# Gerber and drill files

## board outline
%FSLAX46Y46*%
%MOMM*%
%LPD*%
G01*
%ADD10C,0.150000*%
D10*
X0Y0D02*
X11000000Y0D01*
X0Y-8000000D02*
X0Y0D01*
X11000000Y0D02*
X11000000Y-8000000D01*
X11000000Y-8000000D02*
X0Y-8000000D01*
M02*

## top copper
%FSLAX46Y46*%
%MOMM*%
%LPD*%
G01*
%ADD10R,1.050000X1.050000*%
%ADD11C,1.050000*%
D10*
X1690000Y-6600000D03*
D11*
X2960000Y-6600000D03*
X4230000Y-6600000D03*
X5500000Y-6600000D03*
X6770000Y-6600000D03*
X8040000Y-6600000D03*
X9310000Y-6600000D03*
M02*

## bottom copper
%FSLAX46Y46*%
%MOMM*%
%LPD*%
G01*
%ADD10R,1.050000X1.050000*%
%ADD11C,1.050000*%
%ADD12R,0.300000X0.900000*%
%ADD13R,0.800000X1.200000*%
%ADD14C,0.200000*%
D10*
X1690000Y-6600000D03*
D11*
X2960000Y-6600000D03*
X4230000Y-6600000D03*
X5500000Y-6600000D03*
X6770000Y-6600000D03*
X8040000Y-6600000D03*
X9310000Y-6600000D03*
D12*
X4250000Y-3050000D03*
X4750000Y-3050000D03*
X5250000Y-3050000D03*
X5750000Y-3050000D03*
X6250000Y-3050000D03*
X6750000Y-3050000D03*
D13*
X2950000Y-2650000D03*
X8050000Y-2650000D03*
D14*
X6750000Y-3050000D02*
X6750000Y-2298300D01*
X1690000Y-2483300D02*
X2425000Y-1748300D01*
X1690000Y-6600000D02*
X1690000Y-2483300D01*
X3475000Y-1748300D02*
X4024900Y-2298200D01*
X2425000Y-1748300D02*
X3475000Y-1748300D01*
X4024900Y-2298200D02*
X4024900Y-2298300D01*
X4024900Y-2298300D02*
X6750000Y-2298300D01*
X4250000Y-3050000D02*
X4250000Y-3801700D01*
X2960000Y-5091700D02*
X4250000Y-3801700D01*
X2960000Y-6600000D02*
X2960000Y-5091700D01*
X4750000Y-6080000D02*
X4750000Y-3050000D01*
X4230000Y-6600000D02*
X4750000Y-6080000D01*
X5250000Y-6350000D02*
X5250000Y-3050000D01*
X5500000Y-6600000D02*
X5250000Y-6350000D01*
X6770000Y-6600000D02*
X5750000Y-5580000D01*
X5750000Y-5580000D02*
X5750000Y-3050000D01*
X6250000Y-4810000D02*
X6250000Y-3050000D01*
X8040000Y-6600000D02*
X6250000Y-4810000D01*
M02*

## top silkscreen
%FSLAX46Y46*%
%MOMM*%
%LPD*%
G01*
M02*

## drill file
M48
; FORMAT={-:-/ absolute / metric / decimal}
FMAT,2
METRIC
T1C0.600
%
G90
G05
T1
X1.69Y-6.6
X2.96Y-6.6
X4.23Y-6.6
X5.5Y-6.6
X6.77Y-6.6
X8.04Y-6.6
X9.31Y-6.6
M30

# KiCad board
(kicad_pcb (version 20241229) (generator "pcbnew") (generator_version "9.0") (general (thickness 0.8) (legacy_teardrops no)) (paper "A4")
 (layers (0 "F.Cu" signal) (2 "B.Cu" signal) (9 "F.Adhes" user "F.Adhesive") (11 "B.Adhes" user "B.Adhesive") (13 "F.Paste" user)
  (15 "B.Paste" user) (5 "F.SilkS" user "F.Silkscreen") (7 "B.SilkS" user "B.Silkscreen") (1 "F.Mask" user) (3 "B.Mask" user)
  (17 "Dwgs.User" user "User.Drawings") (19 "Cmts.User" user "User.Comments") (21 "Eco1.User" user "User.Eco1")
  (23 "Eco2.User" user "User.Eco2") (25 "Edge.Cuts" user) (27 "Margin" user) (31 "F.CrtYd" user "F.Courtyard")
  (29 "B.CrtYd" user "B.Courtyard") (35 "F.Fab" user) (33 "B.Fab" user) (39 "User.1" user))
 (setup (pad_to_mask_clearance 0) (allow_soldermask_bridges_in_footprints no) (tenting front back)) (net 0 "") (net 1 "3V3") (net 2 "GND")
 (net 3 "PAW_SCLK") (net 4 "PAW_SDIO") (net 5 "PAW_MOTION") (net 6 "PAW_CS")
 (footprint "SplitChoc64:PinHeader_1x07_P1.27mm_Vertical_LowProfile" (layer "F.Cu") (at 0 0)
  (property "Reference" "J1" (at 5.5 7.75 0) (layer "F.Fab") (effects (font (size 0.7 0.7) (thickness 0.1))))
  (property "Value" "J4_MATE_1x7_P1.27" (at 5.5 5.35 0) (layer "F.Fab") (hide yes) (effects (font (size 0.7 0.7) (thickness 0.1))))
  (pad "1" thru_hole rect (at 1.69 6.6) (size 1.05 1.05) (drill 0.6) (layers "*.Cu" "*.Mask") (remove_unused_layers no) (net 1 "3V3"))
  (pad "2" thru_hole circle (at 2.96 6.6) (size 1.05 1.05) (drill 0.6) (layers "*.Cu" "*.Mask") (remove_unused_layers no) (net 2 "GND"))
  (pad "3" thru_hole circle (at 4.23 6.6) (size 1.05 1.05) (drill 0.6) (layers "*.Cu" "*.Mask") (remove_unused_layers no) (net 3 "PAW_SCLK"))
  (pad "4" thru_hole circle (at 5.5 6.6) (size 1.05 1.05) (drill 0.6) (layers "*.Cu" "*.Mask") (remove_unused_layers no) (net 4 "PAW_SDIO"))
  (pad "5" thru_hole circle (at 6.77 6.6) (size 1.05 1.05) (drill 0.6) (layers "*.Cu" "*.Mask") (remove_unused_layers no)
   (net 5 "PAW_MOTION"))
  (pad "6" thru_hole circle (at 8.04 6.6) (size 1.05 1.05) (drill 0.6) (layers "*.Cu" "*.Mask") (remove_unused_layers no) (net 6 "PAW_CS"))
  (pad "7" thru_hole circle (at 9.31 6.6) (size 1.05 1.05) (drill 0.6) (layers "*.Cu" "*.Mask") (remove_unused_layers no)))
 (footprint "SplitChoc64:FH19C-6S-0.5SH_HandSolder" (layer "B.Cu") (at 0 0)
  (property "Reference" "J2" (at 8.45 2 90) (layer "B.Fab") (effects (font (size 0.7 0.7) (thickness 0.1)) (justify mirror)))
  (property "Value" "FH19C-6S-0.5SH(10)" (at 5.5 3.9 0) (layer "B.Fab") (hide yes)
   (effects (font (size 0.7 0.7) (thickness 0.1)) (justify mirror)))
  (pad "1" smd rect (at 4.25 3.05) (size 0.3 0.9) (layers "B.Cu" "B.Mask" "B.Paste") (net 2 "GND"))
  (pad "2" smd rect (at 4.75 3.05) (size 0.3 0.9) (layers "B.Cu" "B.Mask" "B.Paste") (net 3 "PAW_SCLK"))
  (pad "3" smd rect (at 5.25 3.05) (size 0.3 0.9) (layers "B.Cu" "B.Mask" "B.Paste") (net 4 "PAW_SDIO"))
  (pad "4" smd rect (at 5.75 3.05) (size 0.3 0.9) (layers "B.Cu" "B.Mask" "B.Paste") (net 5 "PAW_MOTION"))
  (pad "5" smd rect (at 6.25 3.05) (size 0.3 0.9) (layers "B.Cu" "B.Mask" "B.Paste") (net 6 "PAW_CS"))
  (pad "6" smd rect (at 6.75 3.05) (size 0.3 0.9) (layers "B.Cu" "B.Mask" "B.Paste") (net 1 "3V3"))
  (pad "MP" smd rect (at 2.95 2.65) (size 0.8 1.2) (layers "B.Cu" "B.Mask" "B.Paste"))
  (pad "MP" smd rect (at 8.05 2.65) (size 0.8 1.2) (layers "B.Cu" "B.Mask" "B.Paste")))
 (gr_line (start 0 0) (end 11 0) (stroke (width 0.15) (type default)) (layer "Edge.Cuts"))
 (gr_line (start 0 8) (end 0 0) (stroke (width 0.15) (type default)) (layer "Edge.Cuts"))
 (gr_line (start 11 0) (end 11 8) (stroke (width 0.15) (type default)) (layer "Edge.Cuts"))
 (gr_line (start 11 8) (end 0 8) (stroke (width 0.15) (type default)) (layer "Edge.Cuts"))
 (segment (start 6.75 3.05) (end 6.75 2.2983) (width 0.2) (layer "B.Cu") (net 1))
 (segment (start 1.69 2.4833) (end 2.425 1.7483) (width 0.2) (layer "B.Cu") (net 1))
 (segment (start 1.69 6.6) (end 1.69 2.4833) (width 0.2) (layer "B.Cu") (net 1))
 (segment (start 3.475 1.7483) (end 4.0249 2.2982) (width 0.2) (layer "B.Cu") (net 1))
 (segment (start 2.425 1.7483) (end 3.475 1.7483) (width 0.2) (layer "B.Cu") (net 1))
 (segment (start 4.0249 2.2982) (end 4.0249 2.2983) (width 0.2) (layer "B.Cu") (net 1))
 (segment (start 4.0249 2.2983) (end 6.75 2.2983) (width 0.2) (layer "B.Cu") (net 1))
 (segment (start 4.25 3.05) (end 4.25 3.8017) (width 0.2) (layer "B.Cu") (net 2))
 (segment (start 2.96 5.0917) (end 4.25 3.8017) (width 0.2) (layer "B.Cu") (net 2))
 (segment (start 2.96 6.6) (end 2.96 5.0917) (width 0.2) (layer "B.Cu") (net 2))
 (segment (start 4.75 6.08) (end 4.75 3.05) (width 0.2) (layer "B.Cu") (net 3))
 (segment (start 4.23 6.6) (end 4.75 6.08) (width 0.2) (layer "B.Cu") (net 3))
 (segment (start 5.25 6.35) (end 5.25 3.05) (width 0.2) (layer "B.Cu") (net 4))
 (segment (start 5.5 6.6) (end 5.25 6.35) (width 0.2) (layer "B.Cu") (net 4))
 (segment (start 6.77 6.6) (end 5.75 5.58) (width 0.2) (layer "B.Cu") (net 5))
 (segment (start 5.75 5.58) (end 5.75 3.05) (width 0.2) (layer "B.Cu") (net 5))
 (segment (start 6.25 4.81) (end 6.25 3.05) (width 0.2) (layer "B.Cu") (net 6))
 (segment (start 8.04 6.6) (end 6.25 4.81) (width 0.2) (layer "B.Cu") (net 6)))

